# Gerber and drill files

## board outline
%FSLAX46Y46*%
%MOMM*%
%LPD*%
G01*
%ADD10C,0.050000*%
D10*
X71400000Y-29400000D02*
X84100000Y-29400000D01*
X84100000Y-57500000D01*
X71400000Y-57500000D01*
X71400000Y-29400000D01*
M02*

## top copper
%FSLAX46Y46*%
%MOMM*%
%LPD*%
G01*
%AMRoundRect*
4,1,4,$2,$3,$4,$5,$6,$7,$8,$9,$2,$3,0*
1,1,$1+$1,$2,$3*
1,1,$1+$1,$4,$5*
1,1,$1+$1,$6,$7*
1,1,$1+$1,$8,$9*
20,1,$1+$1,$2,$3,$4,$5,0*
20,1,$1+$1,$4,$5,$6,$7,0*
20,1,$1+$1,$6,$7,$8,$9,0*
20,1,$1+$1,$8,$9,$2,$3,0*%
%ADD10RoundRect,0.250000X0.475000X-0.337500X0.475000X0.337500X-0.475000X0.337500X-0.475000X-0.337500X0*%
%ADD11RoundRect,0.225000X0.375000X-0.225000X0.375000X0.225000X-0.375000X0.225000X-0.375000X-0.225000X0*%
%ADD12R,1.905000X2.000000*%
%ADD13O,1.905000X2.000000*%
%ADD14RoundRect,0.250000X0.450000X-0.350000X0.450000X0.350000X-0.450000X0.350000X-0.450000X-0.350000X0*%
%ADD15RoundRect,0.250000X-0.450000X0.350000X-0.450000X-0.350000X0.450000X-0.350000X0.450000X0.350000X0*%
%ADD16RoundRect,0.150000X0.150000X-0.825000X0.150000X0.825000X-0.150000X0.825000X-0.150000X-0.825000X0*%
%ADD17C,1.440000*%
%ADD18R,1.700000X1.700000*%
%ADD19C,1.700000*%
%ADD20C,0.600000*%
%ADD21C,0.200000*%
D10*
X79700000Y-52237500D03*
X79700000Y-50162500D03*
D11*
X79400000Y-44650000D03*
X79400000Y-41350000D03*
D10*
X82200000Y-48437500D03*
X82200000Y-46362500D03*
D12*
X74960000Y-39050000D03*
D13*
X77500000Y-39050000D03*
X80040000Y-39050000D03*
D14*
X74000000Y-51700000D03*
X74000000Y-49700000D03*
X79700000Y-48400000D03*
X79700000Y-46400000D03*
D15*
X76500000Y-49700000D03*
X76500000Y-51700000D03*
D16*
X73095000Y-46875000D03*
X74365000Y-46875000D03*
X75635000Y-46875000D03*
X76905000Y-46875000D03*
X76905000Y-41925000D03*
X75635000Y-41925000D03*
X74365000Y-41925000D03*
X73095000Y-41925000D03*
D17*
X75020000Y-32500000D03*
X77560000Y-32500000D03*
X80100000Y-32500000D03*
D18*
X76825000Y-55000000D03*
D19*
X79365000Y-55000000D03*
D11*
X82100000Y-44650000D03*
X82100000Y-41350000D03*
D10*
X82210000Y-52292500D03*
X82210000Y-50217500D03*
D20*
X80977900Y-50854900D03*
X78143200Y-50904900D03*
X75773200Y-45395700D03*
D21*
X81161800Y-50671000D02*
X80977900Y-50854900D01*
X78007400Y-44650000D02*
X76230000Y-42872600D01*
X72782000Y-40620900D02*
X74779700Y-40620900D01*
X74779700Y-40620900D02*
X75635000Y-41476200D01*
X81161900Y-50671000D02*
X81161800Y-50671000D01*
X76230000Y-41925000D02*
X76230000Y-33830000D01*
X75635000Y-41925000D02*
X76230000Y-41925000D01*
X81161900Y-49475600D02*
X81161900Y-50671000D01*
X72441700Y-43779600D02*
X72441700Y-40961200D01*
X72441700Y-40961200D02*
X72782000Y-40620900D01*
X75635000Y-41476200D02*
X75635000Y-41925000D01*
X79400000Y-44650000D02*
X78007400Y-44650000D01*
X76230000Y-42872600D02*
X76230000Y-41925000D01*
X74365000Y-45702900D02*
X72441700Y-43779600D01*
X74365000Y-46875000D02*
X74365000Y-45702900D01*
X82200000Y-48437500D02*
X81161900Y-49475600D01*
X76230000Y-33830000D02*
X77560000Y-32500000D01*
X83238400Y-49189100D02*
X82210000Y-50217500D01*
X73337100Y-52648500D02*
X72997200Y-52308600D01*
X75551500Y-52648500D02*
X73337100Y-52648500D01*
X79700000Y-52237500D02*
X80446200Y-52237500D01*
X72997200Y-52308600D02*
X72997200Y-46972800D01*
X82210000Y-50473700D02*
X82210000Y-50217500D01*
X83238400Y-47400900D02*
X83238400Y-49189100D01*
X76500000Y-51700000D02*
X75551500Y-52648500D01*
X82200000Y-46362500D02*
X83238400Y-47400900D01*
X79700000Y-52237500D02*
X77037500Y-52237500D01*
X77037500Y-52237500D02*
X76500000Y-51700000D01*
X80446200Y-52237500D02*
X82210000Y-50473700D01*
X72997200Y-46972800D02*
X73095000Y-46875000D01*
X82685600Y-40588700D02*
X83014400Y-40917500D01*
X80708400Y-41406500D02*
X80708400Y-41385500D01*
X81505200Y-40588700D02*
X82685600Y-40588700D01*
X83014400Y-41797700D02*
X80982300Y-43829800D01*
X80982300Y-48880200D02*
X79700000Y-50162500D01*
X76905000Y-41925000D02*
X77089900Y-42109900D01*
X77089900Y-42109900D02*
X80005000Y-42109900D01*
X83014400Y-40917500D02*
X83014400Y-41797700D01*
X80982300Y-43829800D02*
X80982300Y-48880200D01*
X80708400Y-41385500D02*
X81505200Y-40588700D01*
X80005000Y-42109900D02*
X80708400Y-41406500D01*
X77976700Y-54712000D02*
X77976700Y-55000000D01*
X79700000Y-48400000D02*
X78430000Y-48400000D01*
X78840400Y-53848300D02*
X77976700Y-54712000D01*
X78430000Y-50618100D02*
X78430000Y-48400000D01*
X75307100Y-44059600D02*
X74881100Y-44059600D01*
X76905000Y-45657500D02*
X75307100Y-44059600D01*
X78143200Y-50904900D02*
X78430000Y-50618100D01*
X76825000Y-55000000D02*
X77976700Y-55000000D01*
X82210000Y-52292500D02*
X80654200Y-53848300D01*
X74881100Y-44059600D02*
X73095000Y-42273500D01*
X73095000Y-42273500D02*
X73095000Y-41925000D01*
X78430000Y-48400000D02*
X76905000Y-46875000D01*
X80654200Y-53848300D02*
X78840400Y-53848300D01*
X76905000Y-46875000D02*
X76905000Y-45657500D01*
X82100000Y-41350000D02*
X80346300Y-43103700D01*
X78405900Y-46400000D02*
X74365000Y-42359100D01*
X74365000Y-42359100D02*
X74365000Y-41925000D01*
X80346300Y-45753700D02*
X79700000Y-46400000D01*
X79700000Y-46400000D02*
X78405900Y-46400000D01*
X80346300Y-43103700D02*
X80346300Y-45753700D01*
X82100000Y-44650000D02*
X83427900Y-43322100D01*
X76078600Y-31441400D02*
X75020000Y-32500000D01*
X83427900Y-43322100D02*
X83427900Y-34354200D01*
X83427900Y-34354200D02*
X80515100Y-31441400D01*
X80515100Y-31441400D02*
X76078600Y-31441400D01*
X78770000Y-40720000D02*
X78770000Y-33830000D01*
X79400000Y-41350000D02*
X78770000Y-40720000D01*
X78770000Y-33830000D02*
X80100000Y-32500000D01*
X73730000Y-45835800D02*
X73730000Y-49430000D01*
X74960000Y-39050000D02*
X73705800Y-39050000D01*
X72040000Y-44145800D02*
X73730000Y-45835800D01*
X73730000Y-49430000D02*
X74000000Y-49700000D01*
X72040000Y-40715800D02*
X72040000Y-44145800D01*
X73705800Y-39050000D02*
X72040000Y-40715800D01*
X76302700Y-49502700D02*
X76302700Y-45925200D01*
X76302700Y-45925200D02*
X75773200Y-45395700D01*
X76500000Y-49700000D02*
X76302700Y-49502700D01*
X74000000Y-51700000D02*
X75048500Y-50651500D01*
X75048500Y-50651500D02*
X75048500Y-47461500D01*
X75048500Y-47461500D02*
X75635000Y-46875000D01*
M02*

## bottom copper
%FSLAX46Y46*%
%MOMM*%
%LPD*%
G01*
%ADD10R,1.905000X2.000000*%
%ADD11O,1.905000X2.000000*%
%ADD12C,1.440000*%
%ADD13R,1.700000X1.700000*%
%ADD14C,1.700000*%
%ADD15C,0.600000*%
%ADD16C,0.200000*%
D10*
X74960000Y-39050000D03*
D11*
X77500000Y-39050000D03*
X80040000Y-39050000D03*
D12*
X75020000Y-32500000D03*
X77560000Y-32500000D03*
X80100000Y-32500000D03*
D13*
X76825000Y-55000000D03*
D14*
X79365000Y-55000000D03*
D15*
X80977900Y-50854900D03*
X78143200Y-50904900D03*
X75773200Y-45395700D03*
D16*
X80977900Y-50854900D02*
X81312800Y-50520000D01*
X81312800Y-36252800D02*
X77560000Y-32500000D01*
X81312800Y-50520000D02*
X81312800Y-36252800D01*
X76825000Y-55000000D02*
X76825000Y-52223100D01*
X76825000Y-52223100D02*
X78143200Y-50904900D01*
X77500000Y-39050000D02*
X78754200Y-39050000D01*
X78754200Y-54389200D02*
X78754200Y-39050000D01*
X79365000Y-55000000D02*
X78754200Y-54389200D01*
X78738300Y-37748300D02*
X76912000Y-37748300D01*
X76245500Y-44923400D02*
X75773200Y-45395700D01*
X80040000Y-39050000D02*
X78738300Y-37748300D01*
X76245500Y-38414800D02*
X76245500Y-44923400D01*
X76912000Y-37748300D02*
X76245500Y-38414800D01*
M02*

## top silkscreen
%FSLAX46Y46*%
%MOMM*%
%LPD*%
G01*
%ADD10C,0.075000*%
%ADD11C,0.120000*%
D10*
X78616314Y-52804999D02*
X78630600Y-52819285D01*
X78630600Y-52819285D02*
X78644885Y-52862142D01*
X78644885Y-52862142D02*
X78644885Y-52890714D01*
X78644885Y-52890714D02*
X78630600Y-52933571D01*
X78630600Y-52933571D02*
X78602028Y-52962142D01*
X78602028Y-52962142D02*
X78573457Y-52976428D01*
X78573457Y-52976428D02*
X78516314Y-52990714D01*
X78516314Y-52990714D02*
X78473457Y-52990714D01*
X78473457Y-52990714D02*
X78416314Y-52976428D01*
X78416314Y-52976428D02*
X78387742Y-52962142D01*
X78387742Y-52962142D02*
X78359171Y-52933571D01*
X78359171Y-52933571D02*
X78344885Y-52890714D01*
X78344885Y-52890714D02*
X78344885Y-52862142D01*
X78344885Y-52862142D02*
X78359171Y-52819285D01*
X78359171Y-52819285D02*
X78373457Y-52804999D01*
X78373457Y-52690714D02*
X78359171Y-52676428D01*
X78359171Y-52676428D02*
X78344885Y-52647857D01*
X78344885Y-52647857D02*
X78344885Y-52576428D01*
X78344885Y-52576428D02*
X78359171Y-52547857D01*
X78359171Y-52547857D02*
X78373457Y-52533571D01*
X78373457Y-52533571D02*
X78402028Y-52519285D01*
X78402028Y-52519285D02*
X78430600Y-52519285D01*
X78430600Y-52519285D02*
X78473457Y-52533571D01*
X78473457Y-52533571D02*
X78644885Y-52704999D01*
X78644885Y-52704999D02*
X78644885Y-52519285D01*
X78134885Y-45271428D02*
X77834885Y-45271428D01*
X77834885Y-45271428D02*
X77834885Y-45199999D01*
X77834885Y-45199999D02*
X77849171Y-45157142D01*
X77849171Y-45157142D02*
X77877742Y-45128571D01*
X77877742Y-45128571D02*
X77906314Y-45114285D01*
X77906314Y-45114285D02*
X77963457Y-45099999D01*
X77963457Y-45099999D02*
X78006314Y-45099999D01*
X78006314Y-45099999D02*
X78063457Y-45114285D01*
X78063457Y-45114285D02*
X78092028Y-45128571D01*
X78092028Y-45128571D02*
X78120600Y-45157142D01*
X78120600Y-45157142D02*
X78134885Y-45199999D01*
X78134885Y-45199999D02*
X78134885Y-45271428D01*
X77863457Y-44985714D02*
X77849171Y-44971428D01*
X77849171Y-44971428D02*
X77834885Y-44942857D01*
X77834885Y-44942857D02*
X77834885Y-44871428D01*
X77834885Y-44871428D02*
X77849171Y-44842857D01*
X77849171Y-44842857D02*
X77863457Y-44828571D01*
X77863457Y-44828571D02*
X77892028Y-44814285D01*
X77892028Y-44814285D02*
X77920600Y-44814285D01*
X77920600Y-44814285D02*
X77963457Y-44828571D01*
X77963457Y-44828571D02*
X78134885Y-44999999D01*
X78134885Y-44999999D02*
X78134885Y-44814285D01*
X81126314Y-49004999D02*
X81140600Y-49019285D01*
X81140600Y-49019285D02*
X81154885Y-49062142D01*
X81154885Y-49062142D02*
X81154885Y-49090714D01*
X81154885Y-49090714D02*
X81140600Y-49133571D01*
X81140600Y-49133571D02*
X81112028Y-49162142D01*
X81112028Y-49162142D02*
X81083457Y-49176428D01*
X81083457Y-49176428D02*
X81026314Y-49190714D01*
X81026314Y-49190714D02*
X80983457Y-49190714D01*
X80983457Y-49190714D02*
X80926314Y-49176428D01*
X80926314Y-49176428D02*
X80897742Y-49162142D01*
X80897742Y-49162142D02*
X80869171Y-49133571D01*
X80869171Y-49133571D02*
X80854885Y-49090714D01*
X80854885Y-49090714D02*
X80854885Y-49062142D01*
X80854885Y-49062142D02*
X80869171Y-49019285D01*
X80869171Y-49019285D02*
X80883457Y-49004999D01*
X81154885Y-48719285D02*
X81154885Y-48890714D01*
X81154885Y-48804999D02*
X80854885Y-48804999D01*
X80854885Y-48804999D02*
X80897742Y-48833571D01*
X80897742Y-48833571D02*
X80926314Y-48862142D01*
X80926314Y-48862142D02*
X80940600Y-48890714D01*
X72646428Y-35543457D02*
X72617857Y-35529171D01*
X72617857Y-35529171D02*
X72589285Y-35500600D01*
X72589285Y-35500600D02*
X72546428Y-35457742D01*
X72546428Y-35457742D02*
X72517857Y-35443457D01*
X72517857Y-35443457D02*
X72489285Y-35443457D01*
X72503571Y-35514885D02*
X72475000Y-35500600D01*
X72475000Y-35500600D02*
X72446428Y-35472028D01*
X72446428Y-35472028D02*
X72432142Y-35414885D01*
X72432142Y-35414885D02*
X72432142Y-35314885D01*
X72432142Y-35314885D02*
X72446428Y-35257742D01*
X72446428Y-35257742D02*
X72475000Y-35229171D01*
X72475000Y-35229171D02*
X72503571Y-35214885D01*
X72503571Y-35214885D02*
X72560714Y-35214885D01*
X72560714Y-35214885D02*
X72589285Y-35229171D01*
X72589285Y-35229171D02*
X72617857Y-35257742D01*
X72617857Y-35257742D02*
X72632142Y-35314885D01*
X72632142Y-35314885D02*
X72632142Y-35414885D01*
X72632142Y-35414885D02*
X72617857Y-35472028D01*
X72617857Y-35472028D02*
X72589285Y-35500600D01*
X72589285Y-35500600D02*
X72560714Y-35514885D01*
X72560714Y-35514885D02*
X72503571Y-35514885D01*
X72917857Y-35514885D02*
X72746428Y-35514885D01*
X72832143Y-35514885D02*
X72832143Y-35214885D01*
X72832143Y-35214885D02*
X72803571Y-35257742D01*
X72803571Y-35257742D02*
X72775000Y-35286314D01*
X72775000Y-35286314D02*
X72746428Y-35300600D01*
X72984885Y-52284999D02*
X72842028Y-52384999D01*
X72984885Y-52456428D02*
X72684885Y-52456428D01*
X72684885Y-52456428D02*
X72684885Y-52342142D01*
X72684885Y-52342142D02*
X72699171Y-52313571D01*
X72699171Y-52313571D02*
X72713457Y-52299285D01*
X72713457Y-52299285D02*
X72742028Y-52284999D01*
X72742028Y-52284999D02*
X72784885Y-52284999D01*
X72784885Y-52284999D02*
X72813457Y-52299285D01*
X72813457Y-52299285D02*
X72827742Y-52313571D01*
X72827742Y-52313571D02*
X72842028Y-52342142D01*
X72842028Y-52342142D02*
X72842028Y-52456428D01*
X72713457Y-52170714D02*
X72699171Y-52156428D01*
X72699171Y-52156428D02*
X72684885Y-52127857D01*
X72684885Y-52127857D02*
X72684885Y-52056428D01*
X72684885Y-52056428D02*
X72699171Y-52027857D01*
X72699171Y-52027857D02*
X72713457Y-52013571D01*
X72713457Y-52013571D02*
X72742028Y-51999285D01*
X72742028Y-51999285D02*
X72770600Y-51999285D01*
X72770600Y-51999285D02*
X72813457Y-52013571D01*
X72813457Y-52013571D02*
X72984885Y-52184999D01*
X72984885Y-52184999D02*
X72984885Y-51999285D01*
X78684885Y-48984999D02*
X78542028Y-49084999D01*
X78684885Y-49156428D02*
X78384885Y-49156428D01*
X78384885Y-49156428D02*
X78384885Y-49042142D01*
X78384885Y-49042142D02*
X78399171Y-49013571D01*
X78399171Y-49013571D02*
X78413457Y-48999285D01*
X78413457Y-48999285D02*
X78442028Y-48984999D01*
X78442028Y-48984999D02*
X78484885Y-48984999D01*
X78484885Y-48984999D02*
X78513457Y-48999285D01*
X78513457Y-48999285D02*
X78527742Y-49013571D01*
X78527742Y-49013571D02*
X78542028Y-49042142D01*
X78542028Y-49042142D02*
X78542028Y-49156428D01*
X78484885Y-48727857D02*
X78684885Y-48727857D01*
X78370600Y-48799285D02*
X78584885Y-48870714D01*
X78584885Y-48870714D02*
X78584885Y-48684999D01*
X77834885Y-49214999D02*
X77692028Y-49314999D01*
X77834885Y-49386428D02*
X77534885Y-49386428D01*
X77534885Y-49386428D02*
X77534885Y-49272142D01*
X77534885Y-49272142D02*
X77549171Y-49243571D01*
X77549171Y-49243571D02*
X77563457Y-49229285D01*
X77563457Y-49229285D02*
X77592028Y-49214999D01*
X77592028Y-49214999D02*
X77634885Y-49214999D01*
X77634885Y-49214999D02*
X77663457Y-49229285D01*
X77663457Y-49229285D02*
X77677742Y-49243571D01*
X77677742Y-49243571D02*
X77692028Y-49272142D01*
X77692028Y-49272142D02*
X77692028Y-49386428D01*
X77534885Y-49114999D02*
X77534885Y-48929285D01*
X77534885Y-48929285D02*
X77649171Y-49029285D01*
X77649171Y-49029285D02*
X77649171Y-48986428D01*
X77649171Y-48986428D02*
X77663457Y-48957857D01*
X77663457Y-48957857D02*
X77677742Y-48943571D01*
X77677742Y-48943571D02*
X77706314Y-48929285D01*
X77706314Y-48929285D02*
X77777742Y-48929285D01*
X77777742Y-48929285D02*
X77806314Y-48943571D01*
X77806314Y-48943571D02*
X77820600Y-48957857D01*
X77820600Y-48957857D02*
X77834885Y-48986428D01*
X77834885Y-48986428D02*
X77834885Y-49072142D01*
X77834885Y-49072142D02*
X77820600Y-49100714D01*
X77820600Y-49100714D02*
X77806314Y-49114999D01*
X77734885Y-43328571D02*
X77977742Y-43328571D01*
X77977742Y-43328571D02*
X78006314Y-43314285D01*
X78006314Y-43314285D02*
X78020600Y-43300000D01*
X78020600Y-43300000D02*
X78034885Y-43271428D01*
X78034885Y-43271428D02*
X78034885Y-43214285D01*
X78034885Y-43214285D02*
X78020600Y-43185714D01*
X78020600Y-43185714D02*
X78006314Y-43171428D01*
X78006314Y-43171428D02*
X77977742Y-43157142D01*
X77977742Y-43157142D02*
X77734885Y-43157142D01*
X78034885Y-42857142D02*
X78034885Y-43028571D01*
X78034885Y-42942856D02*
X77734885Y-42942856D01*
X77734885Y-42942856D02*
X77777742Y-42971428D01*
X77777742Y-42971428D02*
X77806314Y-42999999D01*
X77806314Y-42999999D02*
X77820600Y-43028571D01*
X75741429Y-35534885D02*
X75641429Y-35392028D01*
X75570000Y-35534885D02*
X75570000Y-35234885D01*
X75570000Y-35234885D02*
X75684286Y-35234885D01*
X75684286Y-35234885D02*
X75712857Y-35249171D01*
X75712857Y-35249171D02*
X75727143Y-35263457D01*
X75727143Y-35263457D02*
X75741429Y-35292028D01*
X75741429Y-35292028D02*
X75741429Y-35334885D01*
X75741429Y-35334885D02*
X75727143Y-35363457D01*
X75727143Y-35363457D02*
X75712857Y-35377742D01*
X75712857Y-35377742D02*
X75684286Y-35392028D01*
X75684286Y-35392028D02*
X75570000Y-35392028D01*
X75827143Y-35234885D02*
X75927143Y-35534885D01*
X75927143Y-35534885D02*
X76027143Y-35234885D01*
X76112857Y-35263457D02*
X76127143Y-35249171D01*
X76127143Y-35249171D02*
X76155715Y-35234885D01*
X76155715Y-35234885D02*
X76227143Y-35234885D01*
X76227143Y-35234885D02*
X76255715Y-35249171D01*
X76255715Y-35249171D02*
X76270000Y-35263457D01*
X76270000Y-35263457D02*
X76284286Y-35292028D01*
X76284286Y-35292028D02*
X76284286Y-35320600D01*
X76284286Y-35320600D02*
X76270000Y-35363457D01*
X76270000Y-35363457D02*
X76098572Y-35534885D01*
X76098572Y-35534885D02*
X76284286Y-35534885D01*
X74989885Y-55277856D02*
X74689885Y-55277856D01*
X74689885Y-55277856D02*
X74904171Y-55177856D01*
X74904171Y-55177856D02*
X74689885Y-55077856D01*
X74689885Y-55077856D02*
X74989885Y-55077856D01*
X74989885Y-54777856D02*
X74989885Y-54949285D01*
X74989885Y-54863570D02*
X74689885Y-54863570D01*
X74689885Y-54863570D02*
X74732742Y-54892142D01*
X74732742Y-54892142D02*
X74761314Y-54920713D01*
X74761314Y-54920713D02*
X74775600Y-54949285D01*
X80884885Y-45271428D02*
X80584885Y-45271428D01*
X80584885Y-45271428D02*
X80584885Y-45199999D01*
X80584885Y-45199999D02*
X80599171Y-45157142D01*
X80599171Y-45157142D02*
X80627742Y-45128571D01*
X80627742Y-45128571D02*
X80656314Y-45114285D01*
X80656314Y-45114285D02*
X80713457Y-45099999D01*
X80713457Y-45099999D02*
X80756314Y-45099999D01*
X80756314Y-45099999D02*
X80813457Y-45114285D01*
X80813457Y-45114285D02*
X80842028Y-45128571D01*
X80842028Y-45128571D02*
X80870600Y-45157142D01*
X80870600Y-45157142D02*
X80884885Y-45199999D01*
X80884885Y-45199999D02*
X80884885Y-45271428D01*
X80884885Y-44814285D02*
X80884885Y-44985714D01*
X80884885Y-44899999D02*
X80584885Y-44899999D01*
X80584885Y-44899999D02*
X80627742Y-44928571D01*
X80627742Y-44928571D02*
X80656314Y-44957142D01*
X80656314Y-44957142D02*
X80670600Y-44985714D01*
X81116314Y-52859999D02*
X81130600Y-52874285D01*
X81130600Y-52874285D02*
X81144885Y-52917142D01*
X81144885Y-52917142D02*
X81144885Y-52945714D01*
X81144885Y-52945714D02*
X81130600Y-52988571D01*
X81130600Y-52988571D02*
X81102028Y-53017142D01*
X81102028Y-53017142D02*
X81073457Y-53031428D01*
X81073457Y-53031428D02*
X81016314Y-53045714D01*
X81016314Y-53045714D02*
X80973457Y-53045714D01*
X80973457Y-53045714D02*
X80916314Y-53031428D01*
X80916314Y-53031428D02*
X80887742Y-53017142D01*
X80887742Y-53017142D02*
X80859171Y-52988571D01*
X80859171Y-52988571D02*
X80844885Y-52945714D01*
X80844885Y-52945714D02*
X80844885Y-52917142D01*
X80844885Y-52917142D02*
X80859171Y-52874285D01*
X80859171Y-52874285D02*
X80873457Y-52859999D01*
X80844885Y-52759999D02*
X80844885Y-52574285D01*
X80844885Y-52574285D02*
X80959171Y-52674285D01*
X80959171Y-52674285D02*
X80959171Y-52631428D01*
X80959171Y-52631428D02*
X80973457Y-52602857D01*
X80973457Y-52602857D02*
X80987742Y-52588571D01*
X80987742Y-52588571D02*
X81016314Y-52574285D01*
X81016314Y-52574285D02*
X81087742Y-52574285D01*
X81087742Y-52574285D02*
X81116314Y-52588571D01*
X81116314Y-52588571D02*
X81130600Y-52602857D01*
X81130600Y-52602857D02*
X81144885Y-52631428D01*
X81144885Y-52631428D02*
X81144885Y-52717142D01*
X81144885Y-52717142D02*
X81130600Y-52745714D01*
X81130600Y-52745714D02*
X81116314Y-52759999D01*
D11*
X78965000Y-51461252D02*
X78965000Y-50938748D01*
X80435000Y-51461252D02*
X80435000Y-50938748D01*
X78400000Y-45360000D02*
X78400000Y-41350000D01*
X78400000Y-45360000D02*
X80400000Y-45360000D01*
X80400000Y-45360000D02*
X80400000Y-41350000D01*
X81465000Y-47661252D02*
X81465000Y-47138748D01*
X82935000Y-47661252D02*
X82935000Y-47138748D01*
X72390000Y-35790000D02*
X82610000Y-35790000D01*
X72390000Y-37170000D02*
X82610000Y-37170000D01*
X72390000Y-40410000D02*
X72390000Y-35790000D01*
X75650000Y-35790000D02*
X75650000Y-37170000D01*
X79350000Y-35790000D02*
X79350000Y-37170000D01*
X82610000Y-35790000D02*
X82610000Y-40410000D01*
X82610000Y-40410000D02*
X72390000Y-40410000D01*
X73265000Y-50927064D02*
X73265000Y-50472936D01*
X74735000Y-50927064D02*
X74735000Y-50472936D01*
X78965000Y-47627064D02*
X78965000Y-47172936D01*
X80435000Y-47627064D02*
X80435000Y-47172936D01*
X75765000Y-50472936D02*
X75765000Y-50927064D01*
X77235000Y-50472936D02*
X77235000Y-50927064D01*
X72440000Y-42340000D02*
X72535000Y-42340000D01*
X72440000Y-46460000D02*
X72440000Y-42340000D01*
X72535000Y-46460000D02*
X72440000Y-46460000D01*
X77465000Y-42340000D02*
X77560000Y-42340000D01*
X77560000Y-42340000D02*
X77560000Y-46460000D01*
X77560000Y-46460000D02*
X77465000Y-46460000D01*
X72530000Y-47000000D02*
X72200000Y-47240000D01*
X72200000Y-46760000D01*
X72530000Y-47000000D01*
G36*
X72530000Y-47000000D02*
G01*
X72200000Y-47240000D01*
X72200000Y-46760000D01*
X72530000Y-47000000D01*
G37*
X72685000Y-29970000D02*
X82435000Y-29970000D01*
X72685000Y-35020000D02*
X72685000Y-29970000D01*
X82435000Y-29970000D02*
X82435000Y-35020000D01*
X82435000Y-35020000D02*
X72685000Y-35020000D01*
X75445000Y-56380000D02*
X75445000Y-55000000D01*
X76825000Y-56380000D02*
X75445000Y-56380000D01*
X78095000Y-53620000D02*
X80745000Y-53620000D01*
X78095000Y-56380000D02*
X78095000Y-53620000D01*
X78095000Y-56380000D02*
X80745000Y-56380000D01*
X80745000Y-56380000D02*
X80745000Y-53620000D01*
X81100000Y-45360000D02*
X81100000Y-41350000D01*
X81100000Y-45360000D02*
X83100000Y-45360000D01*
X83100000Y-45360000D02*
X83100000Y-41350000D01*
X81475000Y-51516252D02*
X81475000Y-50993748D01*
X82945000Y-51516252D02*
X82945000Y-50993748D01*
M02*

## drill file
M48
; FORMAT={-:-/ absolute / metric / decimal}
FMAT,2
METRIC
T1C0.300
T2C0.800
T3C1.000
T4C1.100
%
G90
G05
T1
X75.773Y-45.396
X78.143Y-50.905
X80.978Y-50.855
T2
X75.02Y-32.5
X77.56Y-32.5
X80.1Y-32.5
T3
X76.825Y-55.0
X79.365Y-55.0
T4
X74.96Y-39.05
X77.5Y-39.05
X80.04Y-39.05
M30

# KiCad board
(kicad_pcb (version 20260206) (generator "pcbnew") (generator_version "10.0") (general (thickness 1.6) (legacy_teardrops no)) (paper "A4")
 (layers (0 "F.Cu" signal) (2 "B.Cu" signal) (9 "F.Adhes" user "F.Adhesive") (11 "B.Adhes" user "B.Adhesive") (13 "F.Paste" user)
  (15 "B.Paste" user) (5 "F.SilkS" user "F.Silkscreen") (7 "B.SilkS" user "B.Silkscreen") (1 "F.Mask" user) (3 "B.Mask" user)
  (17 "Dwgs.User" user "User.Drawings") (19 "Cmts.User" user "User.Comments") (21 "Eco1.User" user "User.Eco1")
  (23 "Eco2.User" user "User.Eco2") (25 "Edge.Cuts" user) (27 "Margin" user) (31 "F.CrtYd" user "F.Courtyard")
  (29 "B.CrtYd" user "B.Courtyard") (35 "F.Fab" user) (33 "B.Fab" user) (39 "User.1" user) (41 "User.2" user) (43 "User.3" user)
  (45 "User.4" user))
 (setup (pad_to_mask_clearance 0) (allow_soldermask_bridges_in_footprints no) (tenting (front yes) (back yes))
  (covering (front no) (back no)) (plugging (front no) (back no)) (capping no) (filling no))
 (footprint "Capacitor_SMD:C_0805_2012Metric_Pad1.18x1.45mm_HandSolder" (layer "F.Cu") (at 79.7 51.2 90)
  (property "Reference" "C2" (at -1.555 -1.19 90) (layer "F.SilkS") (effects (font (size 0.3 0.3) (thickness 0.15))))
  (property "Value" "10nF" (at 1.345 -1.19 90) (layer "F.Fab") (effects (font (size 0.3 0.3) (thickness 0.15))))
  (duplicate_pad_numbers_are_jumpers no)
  (fp_line (start -0.261252 -0.735) (end 0.261252 -0.735) (stroke (width 0.12) (type solid)) (layer "F.SilkS"))
  (fp_line (start -0.261252 0.735) (end 0.261252 0.735) (stroke (width 0.12) (type solid)) (layer "F.SilkS"))
  (pad "1" smd roundrect (at -1.0375 0 90) (size 1.175 1.45) (layers "F.Cu" "F.Mask" "F.Paste") (roundrect_rratio 0.212766) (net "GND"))
  (pad "2" smd roundrect (at 1.0375 0 90) (size 1.175 1.45) (layers "F.Cu" "F.Mask" "F.Paste") (roundrect_rratio 0.212766)
   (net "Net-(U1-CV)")))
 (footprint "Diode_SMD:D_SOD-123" (layer "F.Cu") (at 79.4 43 90)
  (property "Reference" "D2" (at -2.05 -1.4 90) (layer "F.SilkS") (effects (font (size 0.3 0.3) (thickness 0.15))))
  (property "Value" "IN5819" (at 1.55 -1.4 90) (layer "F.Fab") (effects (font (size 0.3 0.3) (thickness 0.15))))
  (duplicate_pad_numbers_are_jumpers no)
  (fp_line (start -2.36 -1) (end 1.65 -1) (stroke (width 0.12) (type solid)) (layer "F.SilkS"))
  (fp_line (start -2.36 -1) (end -2.36 1) (stroke (width 0.12) (type solid)) (layer "F.SilkS"))
  (fp_line (start -2.36 1) (end 1.65 1) (stroke (width 0.12) (type solid)) (layer "F.SilkS"))
  (pad "1" smd roundrect (at -1.65 0 90) (size 0.9 1.2) (layers "F.Cu" "F.Mask" "F.Paste") (roundrect_rratio 0.25) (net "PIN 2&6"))
  (pad "2" smd roundrect (at 1.65 0 90) (size 0.9 1.2) (layers "F.Cu" "F.Mask" "F.Paste") (roundrect_rratio 0.25) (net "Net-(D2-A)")))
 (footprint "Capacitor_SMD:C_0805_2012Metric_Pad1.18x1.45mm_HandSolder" (layer "F.Cu") (at 82.2 47.4 90)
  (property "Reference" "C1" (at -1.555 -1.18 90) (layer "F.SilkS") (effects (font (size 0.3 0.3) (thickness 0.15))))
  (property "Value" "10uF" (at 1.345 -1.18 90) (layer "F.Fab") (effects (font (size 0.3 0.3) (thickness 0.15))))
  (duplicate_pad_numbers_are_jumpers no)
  (fp_line (start -0.261252 -0.735) (end 0.261252 -0.735) (stroke (width 0.12) (type solid)) (layer "F.SilkS"))
  (fp_line (start -0.261252 0.735) (end 0.261252 0.735) (stroke (width 0.12) (type solid)) (layer "F.SilkS"))
  (pad "1" smd roundrect (at -1.0375 0 90) (size 1.175 1.45) (layers "F.Cu" "F.Mask" "F.Paste") (roundrect_rratio 0.212766) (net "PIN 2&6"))
  (pad "2" smd roundrect (at 1.0375 0 90) (size 1.175 1.45) (layers "F.Cu" "F.Mask" "F.Paste") (roundrect_rratio 0.212766) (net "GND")))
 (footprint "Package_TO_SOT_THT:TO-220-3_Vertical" (layer "F.Cu") (at 74.96 39.05)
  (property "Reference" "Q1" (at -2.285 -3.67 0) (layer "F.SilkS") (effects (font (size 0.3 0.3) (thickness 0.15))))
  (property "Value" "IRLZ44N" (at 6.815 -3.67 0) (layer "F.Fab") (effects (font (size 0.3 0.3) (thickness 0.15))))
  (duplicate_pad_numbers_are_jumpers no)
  (fp_line (start -2.57 -3.26) (end 7.65 -3.26) (stroke (width 0.12) (type solid)) (layer "F.SilkS"))
  (fp_line (start -2.57 -1.88) (end 7.65 -1.88) (stroke (width 0.12) (type solid)) (layer "F.SilkS"))
  (fp_line (start -2.57 1.36) (end -2.57 -3.26) (stroke (width 0.12) (type solid)) (layer "F.SilkS"))
  (fp_line (start 0.69 -3.26) (end 0.69 -1.88) (stroke (width 0.12) (type solid)) (layer "F.SilkS"))
  (fp_line (start 4.39 -3.26) (end 4.39 -1.88) (stroke (width 0.12) (type solid)) (layer "F.SilkS"))
  (fp_line (start 7.65 -3.26) (end 7.65 1.36) (stroke (width 0.12) (type solid)) (layer "F.SilkS"))
  (fp_line (start 7.65 1.36) (end -2.57 1.36) (stroke (width 0.12) (type solid)) (layer "F.SilkS"))
  (pad "1" thru_hole rect (at 0 0) (size 1.905 2) (drill 1.1) (layers "*.Cu" "*.Mask") (remove_unused_layers no) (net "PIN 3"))
  (pad "2" thru_hole oval (at 2.54 0) (size 1.905 2) (drill 1.1) (layers "*.Cu" "*.Mask") (remove_unused_layers no) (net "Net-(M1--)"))
  (pad "3" thru_hole oval (at 5.08 0) (size 1.905 2) (drill 1.1) (layers "*.Cu" "*.Mask") (remove_unused_layers no) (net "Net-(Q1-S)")))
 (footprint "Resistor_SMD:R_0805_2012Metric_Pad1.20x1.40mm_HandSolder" (layer "F.Cu") (at 74 50.7 90)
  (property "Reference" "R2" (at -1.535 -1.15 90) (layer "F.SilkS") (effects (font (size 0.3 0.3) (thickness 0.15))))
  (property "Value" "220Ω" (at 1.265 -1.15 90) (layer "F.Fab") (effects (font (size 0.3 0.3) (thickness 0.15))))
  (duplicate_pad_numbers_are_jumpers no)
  (fp_line (start -0.227064 -0.735) (end 0.227064 -0.735) (stroke (width 0.12) (type solid)) (layer "F.SilkS"))
  (fp_line (start -0.227064 0.735) (end 0.227064 0.735) (stroke (width 0.12) (type solid)) (layer "F.SilkS"))
  (pad "1" smd roundrect (at -1 0 90) (size 1.2 1.4) (layers "F.Cu" "F.Mask" "F.Paste") (roundrect_rratio 0.208333) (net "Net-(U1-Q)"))
  (pad "2" smd roundrect (at 1 0 90) (size 1.2 1.4) (layers "F.Cu" "F.Mask" "F.Paste") (roundrect_rratio 0.208333) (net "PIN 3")))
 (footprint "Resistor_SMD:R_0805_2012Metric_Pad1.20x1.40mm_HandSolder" (layer "F.Cu") (at 79.7 47.4 90)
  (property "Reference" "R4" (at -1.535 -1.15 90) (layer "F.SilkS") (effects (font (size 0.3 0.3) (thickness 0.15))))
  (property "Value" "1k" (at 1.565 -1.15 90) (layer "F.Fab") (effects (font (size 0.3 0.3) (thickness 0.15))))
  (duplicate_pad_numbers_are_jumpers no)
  (fp_line (start -0.227064 -0.735) (end 0.227064 -0.735) (stroke (width 0.12) (type solid)) (layer "F.SilkS"))
  (fp_line (start -0.227064 0.735) (end 0.227064 0.735) (stroke (width 0.12) (type solid)) (layer "F.SilkS"))
  (pad "1" smd roundrect (at -1 0 90) (size 1.2 1.4) (layers "F.Cu" "F.Mask" "F.Paste") (roundrect_rratio 0.208333) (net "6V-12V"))
  (pad "2" smd roundrect (at 1 0 90) (size 1.2 1.4) (layers "F.Cu" "F.Mask" "F.Paste") (roundrect_rratio 0.208333) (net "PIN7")))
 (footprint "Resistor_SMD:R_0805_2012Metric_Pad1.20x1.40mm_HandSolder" (layer "F.Cu") (at 76.5 50.7 -90)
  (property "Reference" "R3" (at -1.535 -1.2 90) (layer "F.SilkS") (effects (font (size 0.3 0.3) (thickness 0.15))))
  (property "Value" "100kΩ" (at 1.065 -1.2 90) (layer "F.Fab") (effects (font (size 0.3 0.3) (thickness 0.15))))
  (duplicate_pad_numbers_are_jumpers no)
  (fp_line (start -0.227064 0.735) (end 0.227064 0.735) (stroke (width 0.12) (type solid)) (layer "F.SilkS"))
  (fp_line (start -0.227064 -0.735) (end 0.227064 -0.735) (stroke (width 0.12) (type solid)) (layer "F.SilkS"))
  (pad "1" smd roundrect (at -1 0 270) (size 1.2 1.4) (layers "F.Cu" "F.Mask" "F.Paste") (roundrect_rratio 0.208333) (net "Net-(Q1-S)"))
  (pad "2" smd roundrect (at 1 0 270) (size 1.2 1.4) (layers "F.Cu" "F.Mask" "F.Paste") (roundrect_rratio 0.208333) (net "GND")))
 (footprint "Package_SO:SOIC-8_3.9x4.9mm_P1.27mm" (layer "F.Cu") (at 75 44.4 90)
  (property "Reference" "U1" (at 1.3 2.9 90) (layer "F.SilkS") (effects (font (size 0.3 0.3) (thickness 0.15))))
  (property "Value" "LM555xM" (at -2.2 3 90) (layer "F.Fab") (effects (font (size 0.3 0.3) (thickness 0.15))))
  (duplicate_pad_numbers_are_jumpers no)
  (fp_line (start 2.06 -2.56) (end 2.06 -2.465) (stroke (width 0.12) (type solid)) (layer "F.SilkS"))
  (fp_line (start -2.06 -2.56) (end 2.06 -2.56) (stroke (width 0.12) (type solid)) (layer "F.SilkS"))
  (fp_line (start -2.06 -2.465) (end -2.06 -2.56) (stroke (width 0.12) (type solid)) (layer "F.SilkS"))
  (fp_line (start 2.06 2.465) (end 2.06 2.56) (stroke (width 0.12) (type solid)) (layer "F.SilkS"))
  (fp_line (start 2.06 2.56) (end -2.06 2.56) (stroke (width 0.12) (type solid)) (layer "F.SilkS"))
  (fp_line (start -2.06 2.56) (end -2.06 2.465) (stroke (width 0.12) (type solid)) (layer "F.SilkS"))
  (fp_poly (pts (xy -2.6 -2.47) (xy -2.84 -2.8) (xy -2.36 -2.8)) (stroke (width 0.12) (type solid)) (fill yes) (layer "F.SilkS"))
  (pad "1" smd roundrect (at -2.475 -1.905 90) (size 1.95 0.6) (layers "F.Cu" "F.Mask" "F.Paste") (roundrect_rratio 0.25) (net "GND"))
  (pad "2" smd roundrect (at -2.475 -0.635 90) (size 1.95 0.6) (layers "F.Cu" "F.Mask" "F.Paste") (roundrect_rratio 0.25) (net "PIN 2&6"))
  (pad "3" smd roundrect (at -2.475 0.635 90) (size 1.95 0.6) (layers "F.Cu" "F.Mask" "F.Paste") (roundrect_rratio 0.25) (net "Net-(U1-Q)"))
  (pad "4" smd roundrect (at -2.475 1.905 90) (size 1.95 0.6) (layers "F.Cu" "F.Mask" "F.Paste") (roundrect_rratio 0.25) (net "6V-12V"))
  (pad "5" smd roundrect (at 2.475 1.905 90) (size 1.95 0.6) (layers "F.Cu" "F.Mask" "F.Paste") (roundrect_rratio 0.25) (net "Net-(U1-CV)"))
  (pad "6" smd roundrect (at 2.475 0.635 90) (size 1.95 0.6) (layers "F.Cu" "F.Mask" "F.Paste") (roundrect_rratio 0.25) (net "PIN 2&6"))
  (pad "7" smd roundrect (at 2.475 -0.635 90) (size 1.95 0.6) (layers "F.Cu" "F.Mask" "F.Paste") (roundrect_rratio 0.25) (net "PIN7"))
  (pad "8" smd roundrect (at 2.475 -1.905 90) (size 1.95 0.6) (layers "F.Cu" "F.Mask" "F.Paste") (roundrect_rratio 0.25) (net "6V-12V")))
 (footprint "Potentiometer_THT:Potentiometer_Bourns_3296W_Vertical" (layer "F.Cu") (at 75.02 32.5 180)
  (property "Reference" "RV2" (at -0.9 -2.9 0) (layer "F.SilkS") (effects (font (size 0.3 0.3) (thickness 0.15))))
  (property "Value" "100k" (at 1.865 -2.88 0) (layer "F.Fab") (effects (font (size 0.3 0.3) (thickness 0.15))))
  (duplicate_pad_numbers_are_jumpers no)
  (fp_line (start 2.335 2.53) (end -7.415 2.53) (stroke (width 0.12) (type solid)) (layer "F.SilkS"))
  (fp_line (start 2.335 -2.52) (end 2.335 2.53) (stroke (width 0.12) (type solid)) (layer "F.SilkS"))
  (fp_line (start -7.415 2.53) (end -7.415 -2.52) (stroke (width 0.12) (type solid)) (layer "F.SilkS"))
  (fp_line (start -7.415 -2.52) (end 2.335 -2.52) (stroke (width 0.12) (type solid)) (layer "F.SilkS"))
  (pad "1" thru_hole circle (at 0 0 180) (size 1.44 1.44) (drill 0.8) (layers "*.Cu" "*.Mask") (remove_unused_layers no) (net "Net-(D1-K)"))
  (pad "2" thru_hole circle (at -2.54 0 180) (size 1.44 1.44) (drill 0.8) (layers "*.Cu" "*.Mask") (remove_unused_layers no) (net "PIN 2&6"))
  (pad "3" thru_hole circle (at -5.08 0 180) (size 1.44 1.44) (drill 0.8) (layers "*.Cu" "*.Mask") (remove_unused_layers no)
   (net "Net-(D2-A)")))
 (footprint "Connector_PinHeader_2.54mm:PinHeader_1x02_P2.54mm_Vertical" (layer "F.Cu") (at 76.825 55 90)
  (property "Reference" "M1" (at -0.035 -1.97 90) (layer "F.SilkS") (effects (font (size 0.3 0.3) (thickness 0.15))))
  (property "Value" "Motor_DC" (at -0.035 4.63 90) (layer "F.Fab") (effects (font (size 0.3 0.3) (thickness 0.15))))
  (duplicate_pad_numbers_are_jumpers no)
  (fp_line (start -1.38 -1.38) (end 0 -1.38) (stroke (width 0.12) (type solid)) (layer "F.SilkS"))
  (fp_line (start -1.38 0) (end -1.38 -1.38) (stroke (width 0.12) (type solid)) (layer "F.SilkS"))
  (fp_line (start 1.38 1.27) (end 1.38 3.92) (stroke (width 0.12) (type solid)) (layer "F.SilkS"))
  (fp_line (start -1.38 1.27) (end 1.38 1.27) (stroke (width 0.12) (type solid)) (layer "F.SilkS"))
  (fp_line (start -1.38 1.27) (end -1.38 3.92) (stroke (width 0.12) (type solid)) (layer "F.SilkS"))
  (fp_line (start -1.38 3.92) (end 1.38 3.92) (stroke (width 0.12) (type solid)) (layer "F.SilkS"))
  (pad "1" thru_hole rect (at 0 0 90) (size 1.7 1.7) (drill 1) (layers "*.Cu" "*.Mask") (remove_unused_layers no) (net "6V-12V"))
  (pad "2" thru_hole circle (at 0 2.54 90) (size 1.7 1.7) (drill 1) (layers "*.Cu" "*.Mask") (remove_unused_layers no) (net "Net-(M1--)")))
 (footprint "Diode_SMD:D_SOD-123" (layer "F.Cu") (at 82.1 43 90)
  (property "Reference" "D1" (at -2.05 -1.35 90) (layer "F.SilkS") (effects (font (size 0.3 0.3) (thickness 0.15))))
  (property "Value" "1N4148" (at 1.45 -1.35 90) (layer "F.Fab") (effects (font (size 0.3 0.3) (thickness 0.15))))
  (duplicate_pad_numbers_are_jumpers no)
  (fp_line (start -2.36 -1) (end 1.65 -1) (stroke (width 0.12) (type solid)) (layer "F.SilkS"))
  (fp_line (start -2.36 -1) (end -2.36 1) (stroke (width 0.12) (type solid)) (layer "F.SilkS"))
  (fp_line (start -2.36 1) (end 1.65 1) (stroke (width 0.12) (type solid)) (layer "F.SilkS"))
  (pad "1" smd roundrect (at -1.65 0 90) (size 0.9 1.2) (layers "F.Cu" "F.Mask" "F.Paste") (roundrect_rratio 0.25) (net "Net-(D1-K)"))
  (pad "2" smd roundrect (at 1.65 0 90) (size 0.9 1.2) (layers "F.Cu" "F.Mask" "F.Paste") (roundrect_rratio 0.25) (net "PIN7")))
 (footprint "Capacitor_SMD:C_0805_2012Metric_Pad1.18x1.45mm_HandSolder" (layer "F.Cu") (at 82.21 51.255 90)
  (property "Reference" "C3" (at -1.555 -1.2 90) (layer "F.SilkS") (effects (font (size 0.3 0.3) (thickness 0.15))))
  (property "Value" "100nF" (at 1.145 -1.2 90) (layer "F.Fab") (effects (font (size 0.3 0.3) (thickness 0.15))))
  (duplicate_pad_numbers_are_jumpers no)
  (fp_line (start -0.261252 -0.735) (end 0.261252 -0.735) (stroke (width 0.12) (type solid)) (layer "F.SilkS"))
  (fp_line (start -0.261252 0.735) (end 0.261252 0.735) (stroke (width 0.12) (type solid)) (layer "F.SilkS"))
  (pad "1" smd roundrect (at -1.0375 0 90) (size 1.175 1.45) (layers "F.Cu" "F.Mask" "F.Paste") (roundrect_rratio 0.212766) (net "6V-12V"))
  (pad "2" smd roundrect (at 1.0375 0 90) (size 1.175 1.45) (layers "F.Cu" "F.Mask" "F.Paste") (roundrect_rratio 0.212766) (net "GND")))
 (gr_rect (start 71.4 29.4) (end 84.1 57.5) (stroke (width 0.05) (type default)) (fill no) (layer "Edge.Cuts"))
 (segment (start 81.1618 50.671) (end 80.9779 50.8549) (width 0.2) (layer "F.Cu") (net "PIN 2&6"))
 (segment (start 78.0074 44.65) (end 76.23 42.8726) (width 0.2) (layer "F.Cu") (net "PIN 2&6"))
 (segment (start 72.782 40.6209) (end 74.7797 40.6209) (width 0.2) (layer "F.Cu") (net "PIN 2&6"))
 (segment (start 74.7797 40.6209) (end 75.635 41.4762) (width 0.2) (layer "F.Cu") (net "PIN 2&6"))
 (segment (start 81.1619 50.671) (end 81.1618 50.671) (width 0.2) (layer "F.Cu") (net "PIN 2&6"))
 (segment (start 76.23 41.925) (end 76.23 33.83) (width 0.2) (layer "F.Cu") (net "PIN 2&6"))
 (segment (start 75.635 41.925) (end 76.23 41.925) (width 0.2) (layer "F.Cu") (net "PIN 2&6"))
 (segment (start 81.1619 49.4756) (end 81.1619 50.671) (width 0.2) (layer "F.Cu") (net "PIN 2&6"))
 (segment (start 72.4417 43.7796) (end 72.4417 40.9612) (width 0.2) (layer "F.Cu") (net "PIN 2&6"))
 (segment (start 72.4417 40.9612) (end 72.782 40.6209) (width 0.2) (layer "F.Cu") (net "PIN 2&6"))
 (segment (start 75.635 41.4762) (end 75.635 41.925) (width 0.2) (layer "F.Cu") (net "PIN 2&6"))
 (segment (start 79.4 44.65) (end 78.0074 44.65) (width 0.2) (layer "F.Cu") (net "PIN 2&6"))
 (segment (start 76.23 42.8726) (end 76.23 41.925) (width 0.2) (layer "F.Cu") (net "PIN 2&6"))
 (segment (start 74.365 45.7029) (end 72.4417 43.7796) (width 0.2) (layer "F.Cu") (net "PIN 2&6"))
 (segment (start 74.365 46.875) (end 74.365 45.7029) (width 0.2) (layer "F.Cu") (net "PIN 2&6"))
 (segment (start 82.2 48.4375) (end 81.1619 49.4756) (width 0.2) (layer "F.Cu") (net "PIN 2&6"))
 (segment (start 76.23 33.83) (end 77.56 32.5) (width 0.2) (layer "F.Cu") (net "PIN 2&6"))
 (via (at 80.9779 50.8549) (size 0.6) (drill 0.3) (layers "F.Cu" "B.Cu") (capping no) (covering (front no) (back no))
  (plugging (front no) (back no)) (filling no) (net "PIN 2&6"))
 (segment (start 80.9779 50.8549) (end 81.3128 50.52) (width 0.2) (layer "B.Cu") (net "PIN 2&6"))
 (segment (start 81.3128 36.2528) (end 77.56 32.5) (width 0.2) (layer "B.Cu") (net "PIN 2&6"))
 (segment (start 81.3128 50.52) (end 81.3128 36.2528) (width 0.2) (layer "B.Cu") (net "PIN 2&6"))
 (segment (start 83.2384 49.1891) (end 82.21 50.2175) (width 0.2) (layer "F.Cu") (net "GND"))
 (segment (start 73.3371 52.6485) (end 72.9972 52.3086) (width 0.2) (layer "F.Cu") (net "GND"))
 (segment (start 75.5515 52.6485) (end 73.3371 52.6485) (width 0.2) (layer "F.Cu") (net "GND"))
 (segment (start 79.7 52.2375) (end 80.4462 52.2375) (width 0.2) (layer "F.Cu") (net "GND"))
 (segment (start 72.9972 52.3086) (end 72.9972 46.9728) (width 0.2) (layer "F.Cu") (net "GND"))
 (segment (start 82.21 50.4737) (end 82.21 50.2175) (width 0.2) (layer "F.Cu") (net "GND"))
 (segment (start 83.2384 47.4009) (end 83.2384 49.1891) (width 0.2) (layer "F.Cu") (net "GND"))
 (segment (start 76.5 51.7) (end 75.5515 52.6485) (width 0.2) (layer "F.Cu") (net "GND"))
 (segment (start 82.2 46.3625) (end 83.2384 47.4009) (width 0.2) (layer "F.Cu") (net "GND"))
 (segment (start 79.7 52.2375) (end 77.0375 52.2375) (width 0.2) (layer "F.Cu") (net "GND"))
 (segment (start 77.0375 52.2375) (end 76.5 51.7) (width 0.2) (layer "F.Cu") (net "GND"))
 (segment (start 80.4462 52.2375) (end 82.21 50.4737) (width 0.2) (layer "F.Cu") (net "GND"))
 (segment (start 72.9972 46.9728) (end 73.095 46.875) (width 0.2) (layer "F.Cu") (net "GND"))
 (segment (start 82.6856 40.5887) (end 83.0144 40.9175) (width 0.2) (layer "F.Cu") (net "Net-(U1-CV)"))
 (segment (start 80.7084 41.4065) (end 80.7084 41.3855) (width 0.2) (layer "F.Cu") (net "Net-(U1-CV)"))
 (segment (start 81.5052 40.5887) (end 82.6856 40.5887) (width 0.2) (layer "F.Cu") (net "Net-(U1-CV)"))
 (segment (start 83.0144 41.7977) (end 80.9823 43.8298) (width 0.2) (layer "F.Cu") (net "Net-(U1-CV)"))
 (segment (start 80.9823 48.8802) (end 79.7 50.1625) (width 0.2) (layer "F.Cu") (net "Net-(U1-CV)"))
 (segment (start 76.905 41.925) (end 77.0899 42.1099) (width 0.2) (layer "F.Cu") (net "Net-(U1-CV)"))
 (segment (start 77.0899 42.1099) (end 80.005 42.1099) (width 0.2) (layer "F.Cu") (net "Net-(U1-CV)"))
 (segment (start 83.0144 40.9175) (end 83.0144 41.7977) (width 0.2) (layer "F.Cu") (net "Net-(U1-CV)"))
 (segment (start 80.9823 43.8298) (end 80.9823 48.8802) (width 0.2) (layer "F.Cu") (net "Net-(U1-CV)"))
 (segment (start 80.7084 41.3855) (end 81.5052 40.5887) (width 0.2) (layer "F.Cu") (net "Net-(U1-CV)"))
 (segment (start 80.005 42.1099) (end 80.7084 41.4065) (width 0.2) (layer "F.Cu") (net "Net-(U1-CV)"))
 (segment (start 77.9767 54.712) (end 77.9767 55) (width 0.2) (layer "F.Cu") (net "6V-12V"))
 (segment (start 79.7 48.4) (end 78.43 48.4) (width 0.2) (layer "F.Cu") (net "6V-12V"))
 (segment (start 78.8404 53.8483) (end 77.9767 54.712) (width 0.2) (layer "F.Cu") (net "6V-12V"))
 (segment (start 78.43 50.6181) (end 78.43 48.4) (width 0.2) (layer "F.Cu") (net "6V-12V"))
 (segment (start 75.3071 44.0596) (end 74.8811 44.0596) (width 0.2) (layer "F.Cu") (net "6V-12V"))
 (segment (start 76.905 45.6575) (end 75.3071 44.0596) (width 0.2) (layer "F.Cu") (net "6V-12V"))
 (segment (start 78.1432 50.9049) (end 78.43 50.6181) (width 0.2) (layer "F.Cu") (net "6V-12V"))
 (segment (start 76.825 55) (end 77.9767 55) (width 0.2) (layer "F.Cu") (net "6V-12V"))
 (segment (start 82.21 52.2925) (end 80.6542 53.8483) (width 0.2) (layer "F.Cu") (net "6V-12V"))
 (segment (start 74.8811 44.0596) (end 73.095 42.2735) (width 0.2) (layer "F.Cu") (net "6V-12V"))
 (segment (start 73.095 42.2735) (end 73.095 41.925) (width 0.2) (layer "F.Cu") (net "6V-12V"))
 (segment (start 78.43 48.4) (end 76.905 46.875) (width 0.2) (layer "F.Cu") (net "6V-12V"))
 (segment (start 80.6542 53.8483) (end 78.8404 53.8483) (width 0.2) (layer "F.Cu") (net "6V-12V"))
 (segment (start 76.905 46.875) (end 76.905 45.6575) (width 0.2) (layer "F.Cu") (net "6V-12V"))
 (via (at 78.1432 50.9049) (size 0.6) (drill 0.3) (layers "F.Cu" "B.Cu") (capping no) (covering (front no) (back no))
  (plugging (front no) (back no)) (filling no) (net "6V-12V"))
 (segment (start 76.825 55) (end 76.825 52.2231) (width 0.2) (layer "B.Cu") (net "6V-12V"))
 (segment (start 76.825 52.2231) (end 78.1432 50.9049) (width 0.2) (layer "B.Cu") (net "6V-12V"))
 (segment (start 82.1 41.35) (end 80.3463 43.1037) (width 0.2) (layer "F.Cu") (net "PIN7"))
 (segment (start 78.4059 46.4) (end 74.365 42.3591) (width 0.2) (layer "F.Cu") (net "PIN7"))
 (segment (start 74.365 42.3591) (end 74.365 41.925) (width 0.2) (layer "F.Cu") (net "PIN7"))
 (segment (start 80.3463 45.7537) (end 79.7 46.4) (width 0.2) (layer "F.Cu") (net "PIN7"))
 (segment (start 79.7 46.4) (end 78.4059 46.4) (width 0.2) (layer "F.Cu") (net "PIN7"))
 (segment (start 80.3463 43.1037) (end 80.3463 45.7537) (width 0.2) (layer "F.Cu") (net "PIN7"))
 (segment (start 82.1 44.65) (end 83.4279 43.3221) (width 0.2) (layer "F.Cu") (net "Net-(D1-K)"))
 (segment (start 76.0786 31.4414) (end 75.02 32.5) (width 0.2) (layer "F.Cu") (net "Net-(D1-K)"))
 (segment (start 83.4279 43.3221) (end 83.4279 34.3542) (width 0.2) (layer "F.Cu") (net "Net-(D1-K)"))
 (segment (start 83.4279 34.3542) (end 80.5151 31.4414) (width 0.2) (layer "F.Cu") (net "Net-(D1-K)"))
 (segment (start 80.5151 31.4414) (end 76.0786 31.4414) (width 0.2) (layer "F.Cu") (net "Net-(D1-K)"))
 (segment (start 78.77 40.72) (end 78.77 33.83) (width 0.2) (layer "F.Cu") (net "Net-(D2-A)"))
 (segment (start 79.4 41.35) (end 78.77 40.72) (width 0.2) (layer "F.Cu") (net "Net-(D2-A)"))
 (segment (start 78.77 33.83) (end 80.1 32.5) (width 0.2) (layer "F.Cu") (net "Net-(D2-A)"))
 (segment (start 77.5 39.05) (end 78.7542 39.05) (width 0.2) (layer "B.Cu") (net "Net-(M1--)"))
 (segment (start 78.7542 54.3892) (end 78.7542 39.05) (width 0.2) (layer "B.Cu") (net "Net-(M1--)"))
 (segment (start 79.365 55) (end 78.7542 54.3892) (width 0.2) (layer "B.Cu") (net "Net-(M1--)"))
 (segment (start 73.73 45.8358) (end 73.73 49.43) (width 0.2) (layer "F.Cu") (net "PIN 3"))
 (segment (start 74.96 39.05) (end 73.7058 39.05) (width 0.2) (layer "F.Cu") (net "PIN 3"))
 (segment (start 72.04 44.1458) (end 73.73 45.8358) (width 0.2) (layer "F.Cu") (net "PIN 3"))
 (segment (start 73.73 49.43) (end 74 49.7) (width 0.2) (layer "F.Cu") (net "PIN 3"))
 (segment (start 72.04 40.7158) (end 72.04 44.1458) (width 0.2) (layer "F.Cu") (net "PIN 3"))
 (segment (start 73.7058 39.05) (end 72.04 40.7158) (width 0.2) (layer "F.Cu") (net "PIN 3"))
 (segment (start 76.3027 49.5027) (end 76.3027 45.9252) (width 0.2) (layer "F.Cu") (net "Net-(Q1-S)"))
 (segment (start 76.3027 45.9252) (end 75.7732 45.3957) (width 0.2) (layer "F.Cu") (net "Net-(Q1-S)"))
 (segment (start 76.5 49.7) (end 76.3027 49.5027) (width 0.2) (layer "F.Cu") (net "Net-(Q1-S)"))
 (via (at 75.7732 45.3957) (size 0.6) (drill 0.3) (layers "F.Cu" "B.Cu") (capping no) (covering (front no) (back no))
  (plugging (front no) (back no)) (filling no) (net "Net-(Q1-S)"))
 (segment (start 78.7383 37.7483) (end 76.912 37.7483) (width 0.2) (layer "B.Cu") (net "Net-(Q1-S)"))
 (segment (start 76.2455 44.9234) (end 75.7732 45.3957) (width 0.2) (layer "B.Cu") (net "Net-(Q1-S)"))
 (segment (start 80.04 39.05) (end 78.7383 37.7483) (width 0.2) (layer "B.Cu") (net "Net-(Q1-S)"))
 (segment (start 76.2455 38.4148) (end 76.2455 44.9234) (width 0.2) (layer "B.Cu") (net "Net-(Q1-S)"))
 (segment (start 76.912 37.7483) (end 76.2455 38.4148) (width 0.2) (layer "B.Cu") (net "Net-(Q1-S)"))
 (segment (start 74 51.7) (end 75.0485 50.6515) (width 0.2) (layer "F.Cu") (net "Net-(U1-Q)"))
 (segment (start 75.0485 50.6515) (end 75.0485 47.4615) (width 0.2) (layer "F.Cu") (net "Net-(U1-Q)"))
 (segment (start 75.0485 47.4615) (end 75.635 46.875) (width 0.2) (layer "F.Cu") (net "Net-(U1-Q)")))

